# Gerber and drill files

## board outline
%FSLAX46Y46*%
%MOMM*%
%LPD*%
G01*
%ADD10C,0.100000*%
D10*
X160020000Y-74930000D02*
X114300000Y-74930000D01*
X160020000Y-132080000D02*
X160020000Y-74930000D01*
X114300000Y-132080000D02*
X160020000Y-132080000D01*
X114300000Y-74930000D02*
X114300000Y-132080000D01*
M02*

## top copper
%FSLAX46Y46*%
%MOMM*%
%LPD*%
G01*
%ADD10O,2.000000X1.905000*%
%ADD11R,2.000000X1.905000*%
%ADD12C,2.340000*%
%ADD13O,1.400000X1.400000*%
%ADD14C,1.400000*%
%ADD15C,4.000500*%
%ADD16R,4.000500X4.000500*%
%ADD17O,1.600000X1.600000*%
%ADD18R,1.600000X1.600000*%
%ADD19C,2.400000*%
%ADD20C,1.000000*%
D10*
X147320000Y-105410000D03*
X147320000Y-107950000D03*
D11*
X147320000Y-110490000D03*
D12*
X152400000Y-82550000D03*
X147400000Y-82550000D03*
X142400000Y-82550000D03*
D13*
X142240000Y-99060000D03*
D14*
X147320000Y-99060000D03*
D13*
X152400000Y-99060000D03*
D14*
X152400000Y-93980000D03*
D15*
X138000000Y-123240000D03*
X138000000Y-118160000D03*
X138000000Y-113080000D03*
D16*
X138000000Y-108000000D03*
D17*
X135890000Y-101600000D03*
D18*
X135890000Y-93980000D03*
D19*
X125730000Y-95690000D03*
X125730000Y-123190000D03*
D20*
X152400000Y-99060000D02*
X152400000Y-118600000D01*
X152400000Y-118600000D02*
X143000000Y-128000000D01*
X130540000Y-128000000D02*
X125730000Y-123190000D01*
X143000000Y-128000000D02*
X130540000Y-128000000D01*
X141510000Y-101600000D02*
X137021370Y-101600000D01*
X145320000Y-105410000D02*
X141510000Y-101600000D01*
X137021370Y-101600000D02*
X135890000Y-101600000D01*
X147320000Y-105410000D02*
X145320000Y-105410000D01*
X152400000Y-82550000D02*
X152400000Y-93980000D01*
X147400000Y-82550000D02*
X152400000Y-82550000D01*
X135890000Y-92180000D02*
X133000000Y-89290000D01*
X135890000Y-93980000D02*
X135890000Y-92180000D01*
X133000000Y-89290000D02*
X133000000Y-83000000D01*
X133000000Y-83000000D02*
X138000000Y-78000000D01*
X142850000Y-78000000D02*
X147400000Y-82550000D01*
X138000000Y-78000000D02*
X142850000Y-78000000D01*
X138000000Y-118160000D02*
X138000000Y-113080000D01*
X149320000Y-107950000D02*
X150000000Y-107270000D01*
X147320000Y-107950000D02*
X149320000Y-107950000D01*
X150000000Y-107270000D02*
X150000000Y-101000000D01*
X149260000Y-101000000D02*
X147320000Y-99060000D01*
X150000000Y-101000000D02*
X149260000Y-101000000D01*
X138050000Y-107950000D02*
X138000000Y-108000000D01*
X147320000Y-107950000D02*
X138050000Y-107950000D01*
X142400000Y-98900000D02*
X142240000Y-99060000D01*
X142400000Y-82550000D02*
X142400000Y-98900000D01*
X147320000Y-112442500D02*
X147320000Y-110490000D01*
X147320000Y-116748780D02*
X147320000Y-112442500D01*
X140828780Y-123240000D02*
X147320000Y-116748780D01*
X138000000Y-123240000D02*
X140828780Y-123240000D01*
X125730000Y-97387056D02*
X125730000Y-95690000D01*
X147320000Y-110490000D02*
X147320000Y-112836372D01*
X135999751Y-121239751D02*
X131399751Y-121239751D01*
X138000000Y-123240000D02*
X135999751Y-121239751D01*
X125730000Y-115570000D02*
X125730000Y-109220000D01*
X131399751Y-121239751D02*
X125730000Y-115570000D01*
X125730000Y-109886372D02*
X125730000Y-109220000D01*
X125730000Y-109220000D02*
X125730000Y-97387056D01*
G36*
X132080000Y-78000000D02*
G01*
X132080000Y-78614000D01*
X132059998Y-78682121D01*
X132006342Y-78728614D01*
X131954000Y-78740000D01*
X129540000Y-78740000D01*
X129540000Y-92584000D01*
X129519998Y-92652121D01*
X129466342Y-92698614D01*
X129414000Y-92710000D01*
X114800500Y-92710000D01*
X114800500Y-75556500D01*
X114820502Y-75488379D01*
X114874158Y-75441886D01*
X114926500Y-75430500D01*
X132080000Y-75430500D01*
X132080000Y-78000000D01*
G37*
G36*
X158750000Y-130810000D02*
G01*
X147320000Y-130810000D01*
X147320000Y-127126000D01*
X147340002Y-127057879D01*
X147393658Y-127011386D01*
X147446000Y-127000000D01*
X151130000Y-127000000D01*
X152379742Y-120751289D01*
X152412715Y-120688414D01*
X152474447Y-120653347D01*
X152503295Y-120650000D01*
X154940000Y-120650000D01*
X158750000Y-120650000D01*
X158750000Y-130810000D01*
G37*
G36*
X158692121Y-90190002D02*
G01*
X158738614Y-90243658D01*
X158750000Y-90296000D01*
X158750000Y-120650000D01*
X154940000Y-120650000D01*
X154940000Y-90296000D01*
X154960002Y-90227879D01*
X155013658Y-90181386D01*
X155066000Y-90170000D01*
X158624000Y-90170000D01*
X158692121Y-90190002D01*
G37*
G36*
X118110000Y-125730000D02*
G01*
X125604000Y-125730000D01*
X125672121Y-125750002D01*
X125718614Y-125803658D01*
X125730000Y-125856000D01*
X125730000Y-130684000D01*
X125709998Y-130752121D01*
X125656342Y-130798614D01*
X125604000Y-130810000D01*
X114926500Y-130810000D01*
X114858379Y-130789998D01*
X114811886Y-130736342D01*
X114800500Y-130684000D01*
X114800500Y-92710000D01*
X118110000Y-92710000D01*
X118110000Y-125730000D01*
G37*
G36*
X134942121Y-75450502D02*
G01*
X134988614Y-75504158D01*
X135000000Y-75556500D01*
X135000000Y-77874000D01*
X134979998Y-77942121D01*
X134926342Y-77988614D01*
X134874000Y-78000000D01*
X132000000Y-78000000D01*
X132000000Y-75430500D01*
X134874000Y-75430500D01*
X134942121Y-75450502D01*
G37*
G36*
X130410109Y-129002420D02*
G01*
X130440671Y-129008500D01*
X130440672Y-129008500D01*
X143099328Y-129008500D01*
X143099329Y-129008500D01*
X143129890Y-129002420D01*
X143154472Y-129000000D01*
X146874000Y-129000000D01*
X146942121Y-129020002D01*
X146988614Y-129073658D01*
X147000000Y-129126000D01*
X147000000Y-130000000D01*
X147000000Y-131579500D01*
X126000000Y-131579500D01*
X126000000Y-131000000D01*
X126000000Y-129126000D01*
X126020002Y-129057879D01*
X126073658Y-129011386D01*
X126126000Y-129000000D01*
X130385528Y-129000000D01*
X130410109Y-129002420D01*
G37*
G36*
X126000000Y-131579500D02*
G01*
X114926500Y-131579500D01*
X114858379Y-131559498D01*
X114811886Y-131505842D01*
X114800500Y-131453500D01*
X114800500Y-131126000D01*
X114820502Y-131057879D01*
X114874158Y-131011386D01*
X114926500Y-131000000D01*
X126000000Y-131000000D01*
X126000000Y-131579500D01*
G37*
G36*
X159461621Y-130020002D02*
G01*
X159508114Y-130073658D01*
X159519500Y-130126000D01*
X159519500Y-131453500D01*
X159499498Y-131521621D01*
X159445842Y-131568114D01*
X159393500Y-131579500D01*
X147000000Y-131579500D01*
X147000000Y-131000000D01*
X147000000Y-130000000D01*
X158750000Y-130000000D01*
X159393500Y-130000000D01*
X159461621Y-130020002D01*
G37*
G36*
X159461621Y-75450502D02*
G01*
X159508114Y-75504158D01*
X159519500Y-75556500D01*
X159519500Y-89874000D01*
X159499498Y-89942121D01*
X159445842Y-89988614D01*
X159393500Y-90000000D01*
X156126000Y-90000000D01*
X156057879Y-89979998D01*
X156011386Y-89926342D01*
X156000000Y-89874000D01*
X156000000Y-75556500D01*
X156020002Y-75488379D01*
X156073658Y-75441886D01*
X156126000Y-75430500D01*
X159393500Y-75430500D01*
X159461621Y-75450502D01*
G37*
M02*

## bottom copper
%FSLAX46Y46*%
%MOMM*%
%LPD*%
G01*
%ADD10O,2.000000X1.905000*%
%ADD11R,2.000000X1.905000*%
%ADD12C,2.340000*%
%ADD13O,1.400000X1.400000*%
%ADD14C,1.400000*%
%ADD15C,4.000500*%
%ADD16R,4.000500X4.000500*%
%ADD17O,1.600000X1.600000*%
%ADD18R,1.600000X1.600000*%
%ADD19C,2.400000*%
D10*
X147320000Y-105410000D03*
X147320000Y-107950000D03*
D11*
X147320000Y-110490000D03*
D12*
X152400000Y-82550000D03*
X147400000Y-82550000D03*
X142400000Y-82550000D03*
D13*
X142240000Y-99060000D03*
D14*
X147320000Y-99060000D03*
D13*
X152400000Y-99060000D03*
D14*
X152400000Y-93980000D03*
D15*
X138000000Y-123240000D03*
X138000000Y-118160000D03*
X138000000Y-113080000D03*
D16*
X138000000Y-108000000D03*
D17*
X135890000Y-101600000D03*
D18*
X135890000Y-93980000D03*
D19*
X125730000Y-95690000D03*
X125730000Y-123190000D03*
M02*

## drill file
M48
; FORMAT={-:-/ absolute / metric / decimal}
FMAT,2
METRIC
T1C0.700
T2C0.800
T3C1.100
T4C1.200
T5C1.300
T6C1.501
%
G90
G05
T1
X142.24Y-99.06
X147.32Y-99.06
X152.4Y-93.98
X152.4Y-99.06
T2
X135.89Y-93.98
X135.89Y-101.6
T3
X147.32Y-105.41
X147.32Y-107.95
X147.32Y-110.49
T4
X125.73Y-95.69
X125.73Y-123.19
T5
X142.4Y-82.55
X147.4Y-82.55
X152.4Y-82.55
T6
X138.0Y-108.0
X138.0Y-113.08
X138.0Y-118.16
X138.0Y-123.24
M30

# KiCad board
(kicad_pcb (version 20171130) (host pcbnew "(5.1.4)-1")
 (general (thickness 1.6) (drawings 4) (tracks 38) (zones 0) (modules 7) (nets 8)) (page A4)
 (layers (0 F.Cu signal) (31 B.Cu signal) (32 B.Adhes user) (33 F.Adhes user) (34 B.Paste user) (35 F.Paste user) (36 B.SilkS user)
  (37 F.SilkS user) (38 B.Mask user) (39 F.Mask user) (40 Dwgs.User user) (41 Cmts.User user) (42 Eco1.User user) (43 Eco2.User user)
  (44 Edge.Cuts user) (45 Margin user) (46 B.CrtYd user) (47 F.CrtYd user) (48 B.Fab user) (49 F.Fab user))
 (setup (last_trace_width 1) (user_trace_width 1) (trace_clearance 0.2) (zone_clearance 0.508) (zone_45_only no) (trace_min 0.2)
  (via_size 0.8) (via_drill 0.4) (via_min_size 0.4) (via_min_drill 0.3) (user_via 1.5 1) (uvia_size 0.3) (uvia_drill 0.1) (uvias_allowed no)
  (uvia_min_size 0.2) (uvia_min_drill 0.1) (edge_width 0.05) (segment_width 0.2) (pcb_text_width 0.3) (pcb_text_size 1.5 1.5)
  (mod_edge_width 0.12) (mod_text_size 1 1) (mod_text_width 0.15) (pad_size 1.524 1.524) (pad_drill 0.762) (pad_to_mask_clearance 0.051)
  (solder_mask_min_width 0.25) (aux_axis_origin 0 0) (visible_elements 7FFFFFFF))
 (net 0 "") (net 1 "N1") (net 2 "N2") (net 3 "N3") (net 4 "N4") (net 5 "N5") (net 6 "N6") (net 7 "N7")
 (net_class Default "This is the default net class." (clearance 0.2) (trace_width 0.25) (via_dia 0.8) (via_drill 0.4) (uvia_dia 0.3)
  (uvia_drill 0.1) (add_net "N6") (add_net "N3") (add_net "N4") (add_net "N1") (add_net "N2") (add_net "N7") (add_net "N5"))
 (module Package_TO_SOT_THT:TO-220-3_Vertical (layer F.Cu) (at 147.32 110.49 90)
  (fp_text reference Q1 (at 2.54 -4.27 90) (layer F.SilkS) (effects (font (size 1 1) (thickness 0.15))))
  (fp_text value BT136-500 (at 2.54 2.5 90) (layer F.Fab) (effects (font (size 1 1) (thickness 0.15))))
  (pad 3 thru_hole oval (at 5.08 0 90) (size 1.905 2) (drill 1.1) (layers *.Cu *.Mask) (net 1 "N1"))
  (pad 2 thru_hole oval (at 2.54 0 90) (size 1.905 2) (drill 1.1) (layers *.Cu *.Mask) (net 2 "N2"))
  (pad 1 thru_hole rect (at 0 0 90) (size 1.905 2) (drill 1.1) (layers *.Cu *.Mask) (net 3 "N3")))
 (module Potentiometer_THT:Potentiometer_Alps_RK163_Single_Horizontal (layer F.Cu) (at 152.4 82.55 90)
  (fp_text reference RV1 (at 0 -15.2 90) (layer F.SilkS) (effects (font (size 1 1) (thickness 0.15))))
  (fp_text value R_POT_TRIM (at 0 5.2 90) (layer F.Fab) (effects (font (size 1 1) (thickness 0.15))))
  (pad 1 thru_hole circle (at 0 0 90) (size 2.34 2.34) (drill 1.3) (layers *.Cu *.Mask) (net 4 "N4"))
  (pad 2 thru_hole circle (at 0 -5 90) (size 2.34 2.34) (drill 1.3) (layers *.Cu *.Mask) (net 4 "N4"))
  (pad 3 thru_hole circle (at 0 -10 90) (size 2.34 2.34) (drill 1.3) (layers *.Cu *.Mask) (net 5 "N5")))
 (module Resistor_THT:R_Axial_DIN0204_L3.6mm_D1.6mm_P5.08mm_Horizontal (layer F.Cu) (at 147.32 99.06 180)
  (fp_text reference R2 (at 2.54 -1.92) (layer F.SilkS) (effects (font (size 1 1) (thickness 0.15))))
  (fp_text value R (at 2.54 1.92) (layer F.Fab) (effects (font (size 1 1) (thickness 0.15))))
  (pad 2 thru_hole oval (at 5.08 0 180) (size 1.4 1.4) (drill 0.7) (layers *.Cu *.Mask) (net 5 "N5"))
  (pad 1 thru_hole circle (at 0 0 180) (size 1.4 1.4) (drill 0.7) (layers *.Cu *.Mask) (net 2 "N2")))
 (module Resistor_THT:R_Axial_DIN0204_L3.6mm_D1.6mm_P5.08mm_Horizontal (layer F.Cu) (at 152.4 93.98 270)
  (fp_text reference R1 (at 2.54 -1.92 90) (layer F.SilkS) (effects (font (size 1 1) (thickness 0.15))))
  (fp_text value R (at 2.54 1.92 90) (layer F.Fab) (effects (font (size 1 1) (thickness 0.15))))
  (pad 2 thru_hole oval (at 5.08 0 270) (size 1.4 1.4) (drill 0.7) (layers *.Cu *.Mask) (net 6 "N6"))
  (pad 1 thru_hole circle (at 0 0 270) (size 1.4 1.4) (drill 0.7) (layers *.Cu *.Mask) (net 4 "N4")))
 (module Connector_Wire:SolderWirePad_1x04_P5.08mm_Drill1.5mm (layer F.Cu) (at 138 108 270)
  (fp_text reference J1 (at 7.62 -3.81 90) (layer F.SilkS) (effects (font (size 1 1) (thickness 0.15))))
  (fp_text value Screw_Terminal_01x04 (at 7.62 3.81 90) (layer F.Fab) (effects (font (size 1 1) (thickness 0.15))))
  (pad 4 thru_hole circle (at 15.24 0 270) (size 4.0005 4.0005) (drill 1.50114) (layers *.Cu *.Mask) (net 3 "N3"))
  (pad 3 thru_hole circle (at 10.16 0 270) (size 4.0005 4.0005) (drill 1.50114) (layers *.Cu *.Mask) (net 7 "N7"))
  (pad 2 thru_hole circle (at 5.08 0 270) (size 4.0005 4.0005) (drill 1.50114) (layers *.Cu *.Mask) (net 7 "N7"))
  (pad 1 thru_hole rect (at 0 0 270) (size 4.0005 4.0005) (drill 1.50114) (layers *.Cu *.Mask) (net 2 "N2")))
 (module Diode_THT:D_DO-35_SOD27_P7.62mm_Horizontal (layer F.Cu) (at 135.89 93.98 270)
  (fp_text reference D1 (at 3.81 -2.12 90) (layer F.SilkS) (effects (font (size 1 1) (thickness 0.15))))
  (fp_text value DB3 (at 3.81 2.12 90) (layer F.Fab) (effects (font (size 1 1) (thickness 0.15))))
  (pad 2 thru_hole oval (at 7.62 0 270) (size 1.6 1.6) (drill 0.8) (layers *.Cu *.Mask) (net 1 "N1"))
  (pad 1 thru_hole rect (at 0 0 270) (size 1.6 1.6) (drill 0.8) (layers *.Cu *.Mask) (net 4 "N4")))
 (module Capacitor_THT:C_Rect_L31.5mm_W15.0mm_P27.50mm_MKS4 (layer F.Cu) (at 125.73 123.19 90)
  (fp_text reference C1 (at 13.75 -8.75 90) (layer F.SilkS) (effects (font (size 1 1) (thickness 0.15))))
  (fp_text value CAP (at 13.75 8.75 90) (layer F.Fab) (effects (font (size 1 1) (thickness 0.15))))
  (pad 2 thru_hole circle (at 27.5 0 90) (size 2.4 2.4) (drill 1.2) (layers *.Cu *.Mask) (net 3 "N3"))
  (pad 1 thru_hole circle (at 0 0 90) (size 2.4 2.4) (drill 1.2) (layers *.Cu *.Mask) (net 6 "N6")))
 (gr_line (start 160.02 74.93) (end 114.3 74.93) (layer Edge.Cuts) (width 0.1))
 (gr_line (start 160.02 132.08) (end 160.02 74.93) (layer Edge.Cuts) (width 0.1))
 (gr_line (start 114.3 132.08) (end 160.02 132.08) (layer Edge.Cuts) (width 0.1))
 (gr_line (start 114.3 74.93) (end 114.3 132.08) (layer Edge.Cuts) (width 0.1))
 (segment (start 152.4 99.06) (end 152.4 118.6) (width 1) (layer F.Cu) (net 6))
 (segment (start 152.4 118.6) (end 143 128) (width 1) (layer F.Cu) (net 6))
 (segment (start 130.54 128) (end 125.73 123.19) (width 1) (layer F.Cu) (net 6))
 (segment (start 143 128) (end 130.54 128) (width 1) (layer F.Cu) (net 6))
 (segment (start 141.51 101.6) (end 137.02137 101.6) (width 1) (layer F.Cu) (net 1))
 (segment (start 145.32 105.41) (end 141.51 101.6) (width 1) (layer F.Cu) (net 1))
 (segment (start 137.02137 101.6) (end 135.89 101.6) (width 1) (layer F.Cu) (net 1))
 (segment (start 147.32 105.41) (end 145.32 105.41) (width 1) (layer F.Cu) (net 1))
 (segment (start 152.4 82.55) (end 152.4 93.98) (width 1) (layer F.Cu) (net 4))
 (segment (start 147.4 82.55) (end 152.4 82.55) (width 1) (layer F.Cu) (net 4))
 (segment (start 135.89 92.18) (end 133 89.29) (width 1) (layer F.Cu) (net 4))
 (segment (start 135.89 93.98) (end 135.89 92.18) (width 1) (layer F.Cu) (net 4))
 (segment (start 133 89.29) (end 133 83) (width 1) (layer F.Cu) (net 4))
 (segment (start 133 83) (end 138 78) (width 1) (layer F.Cu) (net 4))
 (segment (start 142.85 78) (end 147.4 82.55) (width 1) (layer F.Cu) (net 4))
 (segment (start 138 78) (end 142.85 78) (width 1) (layer F.Cu) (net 4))
 (segment (start 138 118.16) (end 138 113.08) (width 1) (layer F.Cu) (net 7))
 (segment (start 149.32 107.95) (end 150 107.27) (width 1) (layer F.Cu) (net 2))
 (segment (start 147.32 107.95) (end 149.32 107.95) (width 1) (layer F.Cu) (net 2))
 (segment (start 150 107.27) (end 150 101) (width 1) (layer F.Cu) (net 2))
 (segment (start 149.26 101) (end 147.32 99.06) (width 1) (layer F.Cu) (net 2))
 (segment (start 150 101) (end 149.26 101) (width 1) (layer F.Cu) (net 2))
 (segment (start 138.05 107.95) (end 138 108) (width 1) (layer F.Cu) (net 2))
 (segment (start 147.32 107.95) (end 138.05 107.95) (width 1) (layer F.Cu) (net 2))
 (segment (start 142.4 98.9) (end 142.24 99.06) (width 1) (layer F.Cu) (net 5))
 (segment (start 142.4 82.55) (end 142.4 98.9) (width 1) (layer F.Cu) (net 5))
 (segment (start 147.32 112.4425) (end 147.32 110.49) (width 1) (layer F.Cu) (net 3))
 (segment (start 147.32 116.74878) (end 147.32 112.4425) (width 1) (layer F.Cu) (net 3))
 (segment (start 140.82878 123.24) (end 147.32 116.74878) (width 1) (layer F.Cu) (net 3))
 (segment (start 138 123.24) (end 140.82878 123.24) (width 1) (layer F.Cu) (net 3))
 (segment (start 125.73 97.387056) (end 125.73 95.69) (width 1) (layer F.Cu) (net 3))
 (segment (start 147.32 110.49) (end 147.32 112.836372) (width 1) (layer F.Cu) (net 3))
 (segment (start 135.999751 121.239751) (end 131.399751 121.239751) (width 1) (layer F.Cu) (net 3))
 (segment (start 138 123.24) (end 135.999751 121.239751) (width 1) (layer F.Cu) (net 3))
 (segment (start 125.73 115.57) (end 125.73 109.22) (width 1) (layer F.Cu) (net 3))
 (segment (start 131.399751 121.239751) (end 125.73 115.57) (width 1) (layer F.Cu) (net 3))
 (segment (start 125.73 109.886372) (end 125.73 109.22) (width 1) (layer F.Cu) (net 3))
 (segment (start 125.73 109.22) (end 125.73 97.387056) (width 1) (layer F.Cu) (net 3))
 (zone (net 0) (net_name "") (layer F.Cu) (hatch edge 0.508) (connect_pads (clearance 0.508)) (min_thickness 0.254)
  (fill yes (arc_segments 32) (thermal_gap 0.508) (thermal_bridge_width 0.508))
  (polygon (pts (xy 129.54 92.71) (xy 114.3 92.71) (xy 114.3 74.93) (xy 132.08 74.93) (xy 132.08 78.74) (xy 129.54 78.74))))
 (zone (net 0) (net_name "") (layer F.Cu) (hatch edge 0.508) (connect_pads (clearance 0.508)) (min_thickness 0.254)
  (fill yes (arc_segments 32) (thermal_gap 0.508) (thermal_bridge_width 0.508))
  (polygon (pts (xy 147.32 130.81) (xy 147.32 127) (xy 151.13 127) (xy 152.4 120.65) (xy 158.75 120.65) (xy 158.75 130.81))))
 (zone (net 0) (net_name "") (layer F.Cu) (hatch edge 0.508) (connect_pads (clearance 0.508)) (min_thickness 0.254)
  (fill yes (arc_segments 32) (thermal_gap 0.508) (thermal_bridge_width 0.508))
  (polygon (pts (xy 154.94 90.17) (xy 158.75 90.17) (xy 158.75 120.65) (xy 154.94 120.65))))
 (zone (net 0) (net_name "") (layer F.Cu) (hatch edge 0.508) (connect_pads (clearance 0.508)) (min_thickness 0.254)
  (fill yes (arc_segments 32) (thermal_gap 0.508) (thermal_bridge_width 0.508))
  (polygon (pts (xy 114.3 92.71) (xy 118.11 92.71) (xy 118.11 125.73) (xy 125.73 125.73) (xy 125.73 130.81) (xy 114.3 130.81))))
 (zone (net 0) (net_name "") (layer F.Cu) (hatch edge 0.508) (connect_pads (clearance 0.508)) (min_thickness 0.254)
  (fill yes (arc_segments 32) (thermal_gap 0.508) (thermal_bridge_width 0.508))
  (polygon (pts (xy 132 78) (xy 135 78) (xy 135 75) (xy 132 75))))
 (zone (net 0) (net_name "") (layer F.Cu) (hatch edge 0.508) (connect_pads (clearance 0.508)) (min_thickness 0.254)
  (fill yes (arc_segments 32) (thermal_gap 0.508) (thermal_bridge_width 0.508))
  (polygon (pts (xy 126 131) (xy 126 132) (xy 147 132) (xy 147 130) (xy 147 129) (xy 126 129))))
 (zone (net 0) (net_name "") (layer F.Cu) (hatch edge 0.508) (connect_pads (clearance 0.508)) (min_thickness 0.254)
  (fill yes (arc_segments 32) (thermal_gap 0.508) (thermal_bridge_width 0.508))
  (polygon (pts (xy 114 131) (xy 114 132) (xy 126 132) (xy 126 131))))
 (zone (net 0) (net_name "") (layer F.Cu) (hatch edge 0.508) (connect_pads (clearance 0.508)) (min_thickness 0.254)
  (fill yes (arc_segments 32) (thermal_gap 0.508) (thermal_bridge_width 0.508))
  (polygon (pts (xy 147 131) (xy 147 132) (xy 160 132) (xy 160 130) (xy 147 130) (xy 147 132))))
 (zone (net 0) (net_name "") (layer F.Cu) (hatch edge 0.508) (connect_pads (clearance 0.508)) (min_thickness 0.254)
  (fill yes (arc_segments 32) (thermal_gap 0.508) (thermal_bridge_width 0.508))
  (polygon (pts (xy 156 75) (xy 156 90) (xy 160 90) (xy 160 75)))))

